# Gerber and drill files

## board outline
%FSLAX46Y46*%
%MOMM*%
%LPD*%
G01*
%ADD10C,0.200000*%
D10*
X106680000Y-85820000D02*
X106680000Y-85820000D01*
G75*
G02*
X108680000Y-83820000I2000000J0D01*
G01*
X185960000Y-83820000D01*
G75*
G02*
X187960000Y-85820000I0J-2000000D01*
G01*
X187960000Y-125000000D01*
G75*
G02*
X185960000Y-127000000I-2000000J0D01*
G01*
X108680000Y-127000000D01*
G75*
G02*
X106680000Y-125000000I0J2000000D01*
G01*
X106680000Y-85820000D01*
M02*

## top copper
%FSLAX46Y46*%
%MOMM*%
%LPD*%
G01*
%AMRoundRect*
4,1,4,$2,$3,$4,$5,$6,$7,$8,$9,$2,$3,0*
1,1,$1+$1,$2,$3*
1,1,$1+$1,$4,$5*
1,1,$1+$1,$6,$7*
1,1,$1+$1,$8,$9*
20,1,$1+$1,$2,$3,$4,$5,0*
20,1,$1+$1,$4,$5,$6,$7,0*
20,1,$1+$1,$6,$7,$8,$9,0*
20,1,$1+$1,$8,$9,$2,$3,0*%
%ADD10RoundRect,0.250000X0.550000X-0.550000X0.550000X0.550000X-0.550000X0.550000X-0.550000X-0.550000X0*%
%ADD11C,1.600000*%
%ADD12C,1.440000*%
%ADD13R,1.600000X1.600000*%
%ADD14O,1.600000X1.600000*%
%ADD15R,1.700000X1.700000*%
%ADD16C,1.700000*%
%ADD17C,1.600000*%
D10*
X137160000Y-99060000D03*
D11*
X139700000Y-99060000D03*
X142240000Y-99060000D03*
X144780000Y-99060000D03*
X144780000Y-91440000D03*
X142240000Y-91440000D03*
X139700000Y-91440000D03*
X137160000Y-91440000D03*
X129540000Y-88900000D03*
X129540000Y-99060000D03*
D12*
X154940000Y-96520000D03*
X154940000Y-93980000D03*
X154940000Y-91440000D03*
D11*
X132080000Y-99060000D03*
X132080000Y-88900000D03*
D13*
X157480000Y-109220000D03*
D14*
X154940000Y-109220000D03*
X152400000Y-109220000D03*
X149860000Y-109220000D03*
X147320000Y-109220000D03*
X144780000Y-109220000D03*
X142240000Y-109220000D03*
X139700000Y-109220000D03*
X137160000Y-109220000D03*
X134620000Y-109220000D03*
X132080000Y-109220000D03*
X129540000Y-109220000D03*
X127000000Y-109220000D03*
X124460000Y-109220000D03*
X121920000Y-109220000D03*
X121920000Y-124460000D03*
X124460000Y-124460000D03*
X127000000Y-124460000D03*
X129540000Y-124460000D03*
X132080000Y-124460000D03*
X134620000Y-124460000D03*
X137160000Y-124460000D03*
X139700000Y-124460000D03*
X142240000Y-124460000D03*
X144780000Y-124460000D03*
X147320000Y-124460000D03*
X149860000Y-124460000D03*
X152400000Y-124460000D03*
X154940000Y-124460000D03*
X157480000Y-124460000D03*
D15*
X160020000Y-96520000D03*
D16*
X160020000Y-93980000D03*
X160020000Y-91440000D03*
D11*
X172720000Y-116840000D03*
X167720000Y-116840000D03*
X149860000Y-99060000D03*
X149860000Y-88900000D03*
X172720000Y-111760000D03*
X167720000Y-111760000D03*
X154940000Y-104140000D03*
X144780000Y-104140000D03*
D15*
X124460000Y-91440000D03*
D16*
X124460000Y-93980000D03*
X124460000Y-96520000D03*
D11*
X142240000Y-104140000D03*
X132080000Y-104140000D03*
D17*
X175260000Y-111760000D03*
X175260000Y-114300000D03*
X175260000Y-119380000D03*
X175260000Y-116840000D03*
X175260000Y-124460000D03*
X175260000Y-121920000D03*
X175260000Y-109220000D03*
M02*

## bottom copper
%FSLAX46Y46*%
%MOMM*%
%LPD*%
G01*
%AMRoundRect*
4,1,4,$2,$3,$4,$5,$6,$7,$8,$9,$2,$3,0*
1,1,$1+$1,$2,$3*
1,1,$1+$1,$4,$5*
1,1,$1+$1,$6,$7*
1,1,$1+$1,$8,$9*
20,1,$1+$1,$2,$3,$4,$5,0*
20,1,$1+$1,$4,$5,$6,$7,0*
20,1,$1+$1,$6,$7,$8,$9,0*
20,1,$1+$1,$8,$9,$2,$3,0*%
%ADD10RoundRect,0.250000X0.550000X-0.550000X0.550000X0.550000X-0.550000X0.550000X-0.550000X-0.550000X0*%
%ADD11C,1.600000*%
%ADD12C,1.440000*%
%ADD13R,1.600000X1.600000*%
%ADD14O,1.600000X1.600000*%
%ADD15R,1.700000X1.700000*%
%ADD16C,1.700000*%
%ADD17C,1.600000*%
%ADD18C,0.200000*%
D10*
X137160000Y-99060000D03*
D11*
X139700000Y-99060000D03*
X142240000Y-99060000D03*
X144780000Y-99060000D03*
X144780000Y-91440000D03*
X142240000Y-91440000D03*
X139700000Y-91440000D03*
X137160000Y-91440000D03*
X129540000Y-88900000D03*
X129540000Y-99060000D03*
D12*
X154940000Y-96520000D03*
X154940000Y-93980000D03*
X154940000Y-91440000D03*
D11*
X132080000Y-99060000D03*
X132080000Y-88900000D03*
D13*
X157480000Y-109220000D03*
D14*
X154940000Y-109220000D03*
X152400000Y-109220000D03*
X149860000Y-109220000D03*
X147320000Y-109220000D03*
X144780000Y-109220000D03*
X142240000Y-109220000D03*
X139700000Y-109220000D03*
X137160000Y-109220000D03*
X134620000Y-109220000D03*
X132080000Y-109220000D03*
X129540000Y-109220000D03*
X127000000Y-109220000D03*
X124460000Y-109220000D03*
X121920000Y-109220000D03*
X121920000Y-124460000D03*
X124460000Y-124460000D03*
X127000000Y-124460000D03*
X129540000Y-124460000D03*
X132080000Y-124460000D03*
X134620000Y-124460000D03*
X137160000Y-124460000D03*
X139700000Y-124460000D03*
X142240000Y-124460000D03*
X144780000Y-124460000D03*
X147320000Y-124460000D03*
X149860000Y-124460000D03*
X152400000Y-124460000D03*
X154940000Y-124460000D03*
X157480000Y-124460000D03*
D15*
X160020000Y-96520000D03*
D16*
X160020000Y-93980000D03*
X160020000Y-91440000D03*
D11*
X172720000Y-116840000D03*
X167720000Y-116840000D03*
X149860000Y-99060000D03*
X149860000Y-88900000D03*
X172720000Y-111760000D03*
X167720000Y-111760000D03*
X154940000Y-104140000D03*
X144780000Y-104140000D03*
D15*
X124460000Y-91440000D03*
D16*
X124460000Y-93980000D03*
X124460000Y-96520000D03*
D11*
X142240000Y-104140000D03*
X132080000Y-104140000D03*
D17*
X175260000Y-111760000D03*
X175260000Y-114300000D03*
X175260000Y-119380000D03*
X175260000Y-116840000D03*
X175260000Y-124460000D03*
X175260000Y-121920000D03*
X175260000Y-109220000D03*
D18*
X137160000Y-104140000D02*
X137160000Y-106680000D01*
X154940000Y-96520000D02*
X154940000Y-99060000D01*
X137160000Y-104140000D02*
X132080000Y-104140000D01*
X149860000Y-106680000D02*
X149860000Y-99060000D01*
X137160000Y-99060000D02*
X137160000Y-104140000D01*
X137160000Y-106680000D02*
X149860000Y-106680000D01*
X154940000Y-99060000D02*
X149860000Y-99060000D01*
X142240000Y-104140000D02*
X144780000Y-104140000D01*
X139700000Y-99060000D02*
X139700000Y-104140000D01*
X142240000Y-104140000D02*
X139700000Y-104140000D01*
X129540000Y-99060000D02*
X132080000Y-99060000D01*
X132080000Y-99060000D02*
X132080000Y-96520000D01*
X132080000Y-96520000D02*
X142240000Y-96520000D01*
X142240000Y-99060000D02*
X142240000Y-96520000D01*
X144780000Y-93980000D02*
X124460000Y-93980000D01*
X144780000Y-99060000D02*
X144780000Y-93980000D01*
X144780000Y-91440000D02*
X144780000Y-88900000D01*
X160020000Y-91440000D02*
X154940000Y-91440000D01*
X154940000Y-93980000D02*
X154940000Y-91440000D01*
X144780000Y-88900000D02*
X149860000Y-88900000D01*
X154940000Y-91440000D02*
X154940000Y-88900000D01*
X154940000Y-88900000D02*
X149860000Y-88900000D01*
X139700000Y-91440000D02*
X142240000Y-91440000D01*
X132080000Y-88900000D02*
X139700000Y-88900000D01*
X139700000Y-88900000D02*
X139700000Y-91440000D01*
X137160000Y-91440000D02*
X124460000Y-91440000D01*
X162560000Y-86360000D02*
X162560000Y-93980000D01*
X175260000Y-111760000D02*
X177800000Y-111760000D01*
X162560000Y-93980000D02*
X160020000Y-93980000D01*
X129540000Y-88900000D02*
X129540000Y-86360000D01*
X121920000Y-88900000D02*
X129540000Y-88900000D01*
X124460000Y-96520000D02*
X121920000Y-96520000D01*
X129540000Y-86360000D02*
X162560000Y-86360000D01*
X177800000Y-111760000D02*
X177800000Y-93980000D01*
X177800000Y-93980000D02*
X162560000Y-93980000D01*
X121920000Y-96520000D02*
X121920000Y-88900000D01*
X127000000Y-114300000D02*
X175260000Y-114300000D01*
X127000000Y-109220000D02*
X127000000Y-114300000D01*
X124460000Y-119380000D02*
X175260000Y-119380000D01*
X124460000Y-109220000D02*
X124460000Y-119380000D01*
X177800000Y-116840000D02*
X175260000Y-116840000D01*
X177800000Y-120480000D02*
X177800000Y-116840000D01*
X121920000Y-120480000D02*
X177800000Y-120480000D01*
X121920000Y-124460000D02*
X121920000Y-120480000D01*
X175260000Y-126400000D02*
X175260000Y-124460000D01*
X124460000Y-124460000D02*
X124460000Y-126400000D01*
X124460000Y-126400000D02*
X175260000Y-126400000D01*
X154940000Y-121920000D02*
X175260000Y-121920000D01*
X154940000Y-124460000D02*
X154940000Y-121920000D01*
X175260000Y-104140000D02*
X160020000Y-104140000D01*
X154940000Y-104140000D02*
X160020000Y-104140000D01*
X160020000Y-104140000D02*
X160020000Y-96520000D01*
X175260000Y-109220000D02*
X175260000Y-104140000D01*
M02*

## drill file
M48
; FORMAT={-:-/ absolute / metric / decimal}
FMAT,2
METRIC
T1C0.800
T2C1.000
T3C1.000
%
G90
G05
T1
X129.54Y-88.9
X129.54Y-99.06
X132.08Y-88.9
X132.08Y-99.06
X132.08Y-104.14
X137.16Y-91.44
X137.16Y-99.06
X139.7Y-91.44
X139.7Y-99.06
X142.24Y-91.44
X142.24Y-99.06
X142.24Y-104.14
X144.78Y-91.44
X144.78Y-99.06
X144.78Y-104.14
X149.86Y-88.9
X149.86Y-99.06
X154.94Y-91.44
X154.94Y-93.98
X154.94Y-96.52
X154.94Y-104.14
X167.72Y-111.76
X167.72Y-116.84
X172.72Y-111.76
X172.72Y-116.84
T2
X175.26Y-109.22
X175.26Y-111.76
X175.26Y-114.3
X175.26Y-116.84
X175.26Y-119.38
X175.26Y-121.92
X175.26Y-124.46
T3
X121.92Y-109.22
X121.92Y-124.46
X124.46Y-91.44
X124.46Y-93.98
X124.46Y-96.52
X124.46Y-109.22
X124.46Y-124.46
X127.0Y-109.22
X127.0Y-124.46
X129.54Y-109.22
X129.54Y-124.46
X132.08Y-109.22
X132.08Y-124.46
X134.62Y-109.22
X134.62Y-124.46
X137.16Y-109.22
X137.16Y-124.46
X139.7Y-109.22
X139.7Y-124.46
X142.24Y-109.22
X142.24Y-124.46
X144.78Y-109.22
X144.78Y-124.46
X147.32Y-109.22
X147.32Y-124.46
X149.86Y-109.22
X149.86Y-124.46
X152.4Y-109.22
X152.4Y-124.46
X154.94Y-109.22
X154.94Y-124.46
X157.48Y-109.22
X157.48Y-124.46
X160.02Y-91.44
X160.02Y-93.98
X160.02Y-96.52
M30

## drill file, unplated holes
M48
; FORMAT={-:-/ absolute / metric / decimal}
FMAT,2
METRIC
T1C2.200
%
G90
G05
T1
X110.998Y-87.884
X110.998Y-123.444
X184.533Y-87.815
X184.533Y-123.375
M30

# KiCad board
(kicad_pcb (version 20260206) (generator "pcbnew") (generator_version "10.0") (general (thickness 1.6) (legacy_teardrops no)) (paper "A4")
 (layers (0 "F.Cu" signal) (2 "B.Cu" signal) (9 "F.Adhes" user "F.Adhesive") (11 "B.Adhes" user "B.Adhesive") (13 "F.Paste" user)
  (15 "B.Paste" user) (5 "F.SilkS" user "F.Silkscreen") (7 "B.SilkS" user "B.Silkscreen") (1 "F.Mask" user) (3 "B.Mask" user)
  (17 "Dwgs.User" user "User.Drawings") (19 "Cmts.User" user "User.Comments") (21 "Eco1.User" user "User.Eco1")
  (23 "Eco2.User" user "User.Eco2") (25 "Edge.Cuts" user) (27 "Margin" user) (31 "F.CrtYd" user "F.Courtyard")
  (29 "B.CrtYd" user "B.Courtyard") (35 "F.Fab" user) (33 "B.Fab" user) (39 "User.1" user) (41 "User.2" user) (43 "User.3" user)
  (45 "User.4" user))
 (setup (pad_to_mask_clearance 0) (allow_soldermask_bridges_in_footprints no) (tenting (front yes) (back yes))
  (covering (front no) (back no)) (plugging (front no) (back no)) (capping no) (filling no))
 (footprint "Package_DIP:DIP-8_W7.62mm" (layer "F.Cu") (at 137.16 99.06 90)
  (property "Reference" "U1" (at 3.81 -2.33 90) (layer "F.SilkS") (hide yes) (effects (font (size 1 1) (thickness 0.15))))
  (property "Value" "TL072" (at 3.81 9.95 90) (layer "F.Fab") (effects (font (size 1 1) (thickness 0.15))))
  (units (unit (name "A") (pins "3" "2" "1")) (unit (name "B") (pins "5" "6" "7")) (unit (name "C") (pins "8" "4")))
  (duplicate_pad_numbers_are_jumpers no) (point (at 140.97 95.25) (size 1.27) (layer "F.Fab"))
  (pad "1" thru_hole roundrect (at 0 0 90) (size 1.6 1.6) (drill 0.8) (layers "*.Cu" "*.Mask") (remove_unused_layers no)
   (roundrect_rratio 0.15625) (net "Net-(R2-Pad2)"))
  (pad "2" thru_hole circle (at 0 2.54 90) (size 1.6 1.6) (drill 0.8) (layers "*.Cu" "*.Mask") (remove_unused_layers no) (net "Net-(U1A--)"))
  (pad "3" thru_hole circle (at 0 5.08 90) (size 1.6 1.6) (drill 0.8) (layers "*.Cu" "*.Mask") (remove_unused_layers no) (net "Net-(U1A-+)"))
  (pad "4" thru_hole circle (at 0 7.62 90) (size 1.6 1.6) (drill 0.8) (layers "*.Cu" "*.Mask") (remove_unused_layers no) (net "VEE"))
  (pad "5" thru_hole circle (at 7.62 7.62 90) (size 1.6 1.6) (drill 0.8) (layers "*.Cu" "*.Mask") (remove_unused_layers no) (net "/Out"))
  (pad "6" thru_hole circle (at 7.62 5.08 90) (size 1.6 1.6) (drill 0.8) (layers "*.Cu" "*.Mask") (remove_unused_layers no)
   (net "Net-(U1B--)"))
  (pad "7" thru_hole circle (at 7.62 2.54 90) (size 1.6 1.6) (drill 0.8) (layers "*.Cu" "*.Mask") (remove_unused_layers no)
   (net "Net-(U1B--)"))
  (pad "8" thru_hole circle (at 7.62 0 90) (size 1.6 1.6) (drill 0.8) (layers "*.Cu" "*.Mask") (remove_unused_layers no) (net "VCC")))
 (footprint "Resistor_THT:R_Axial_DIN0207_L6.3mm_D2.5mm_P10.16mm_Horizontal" (layer "F.Cu") (at 129.54 88.9 -90)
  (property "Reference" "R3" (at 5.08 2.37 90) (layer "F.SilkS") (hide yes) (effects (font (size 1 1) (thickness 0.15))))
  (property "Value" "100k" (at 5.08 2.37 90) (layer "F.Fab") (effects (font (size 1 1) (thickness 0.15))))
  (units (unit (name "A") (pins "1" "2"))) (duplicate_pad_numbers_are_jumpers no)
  (pad "1" thru_hole circle (at 0 0 270) (size 1.6 1.6) (drill 0.8) (layers "*.Cu" "*.Mask") (remove_unused_layers no) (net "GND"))
  (pad "2" thru_hole circle (at 10.16 0 270) (size 1.6 1.6) (drill 0.8) (layers "*.Cu" "*.Mask") (remove_unused_layers no)
   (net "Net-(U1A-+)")))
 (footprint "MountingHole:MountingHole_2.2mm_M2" (layer "F.Cu") (at 110.998 123.444)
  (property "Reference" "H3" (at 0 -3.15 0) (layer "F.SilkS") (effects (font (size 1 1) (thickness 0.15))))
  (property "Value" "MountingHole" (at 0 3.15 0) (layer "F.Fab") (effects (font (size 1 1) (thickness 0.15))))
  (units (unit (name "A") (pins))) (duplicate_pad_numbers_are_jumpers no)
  (pad "" np_thru_hole circle (at 0 0) (size 2.2 2.2) (drill 2.2) (layers "*.Cu" "*.Mask")))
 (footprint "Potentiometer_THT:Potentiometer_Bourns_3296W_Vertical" (layer "F.Cu") (at 154.94 96.52 -90)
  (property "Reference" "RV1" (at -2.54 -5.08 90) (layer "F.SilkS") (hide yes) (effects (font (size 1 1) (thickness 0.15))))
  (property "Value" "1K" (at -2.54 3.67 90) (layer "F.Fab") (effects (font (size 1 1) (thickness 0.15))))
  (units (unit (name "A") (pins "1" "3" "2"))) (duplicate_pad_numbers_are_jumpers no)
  (pad "1" thru_hole circle (at 0 0 270) (size 1.44 1.44) (drill 0.8) (layers "*.Cu" "*.Mask") (remove_unused_layers no)
   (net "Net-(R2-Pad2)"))
  (pad "2" thru_hole circle (at -2.54 0 270) (size 1.44 1.44) (drill 0.8) (layers "*.Cu" "*.Mask") (remove_unused_layers no) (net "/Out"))
  (pad "3" thru_hole circle (at -5.08 0 270) (size 1.44 1.44) (drill 0.8) (layers "*.Cu" "*.Mask") (remove_unused_layers no) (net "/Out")))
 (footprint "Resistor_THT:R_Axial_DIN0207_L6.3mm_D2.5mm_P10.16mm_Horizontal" (layer "F.Cu") (at 132.08 99.06 90)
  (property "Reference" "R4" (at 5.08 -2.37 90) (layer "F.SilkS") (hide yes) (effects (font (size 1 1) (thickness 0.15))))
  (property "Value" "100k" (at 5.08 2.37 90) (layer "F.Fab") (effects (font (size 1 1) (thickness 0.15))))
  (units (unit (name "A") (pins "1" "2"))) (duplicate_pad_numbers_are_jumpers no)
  (pad "1" thru_hole circle (at 0 0 90) (size 1.6 1.6) (drill 0.8) (layers "*.Cu" "*.Mask") (remove_unused_layers no) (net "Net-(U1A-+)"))
  (pad "2" thru_hole circle (at 10.16 0 90) (size 1.6 1.6) (drill 0.8) (layers "*.Cu" "*.Mask") (remove_unused_layers no)
   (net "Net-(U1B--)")))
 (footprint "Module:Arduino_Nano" (layer "F.Cu") (at 157.48 109.22 -90)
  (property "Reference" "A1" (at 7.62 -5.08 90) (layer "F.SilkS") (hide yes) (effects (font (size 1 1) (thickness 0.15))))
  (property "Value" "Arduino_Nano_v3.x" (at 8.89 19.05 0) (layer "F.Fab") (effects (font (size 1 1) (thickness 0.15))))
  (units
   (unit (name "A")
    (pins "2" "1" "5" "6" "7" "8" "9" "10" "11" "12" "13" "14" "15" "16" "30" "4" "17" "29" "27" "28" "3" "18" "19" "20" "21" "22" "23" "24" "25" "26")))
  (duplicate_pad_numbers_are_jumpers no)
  (pad "1" thru_hole rect (at 0 0 270) (size 1.6 1.6) (drill 1) (layers "*.Cu" "*.Mask") (remove_unused_layers no)
   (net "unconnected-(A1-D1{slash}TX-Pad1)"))
  (pad "2" thru_hole oval (at 0 2.54 270) (size 1.6 1.6) (drill 1) (layers "*.Cu" "*.Mask") (remove_unused_layers no)
   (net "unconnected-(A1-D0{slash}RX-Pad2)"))
  (pad "3" thru_hole oval (at 0 5.08 270) (size 1.6 1.6) (drill 1) (layers "*.Cu" "*.Mask") (remove_unused_layers no)
   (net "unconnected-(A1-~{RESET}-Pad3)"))
  (pad "4" thru_hole oval (at 0 7.62 270) (size 1.6 1.6) (drill 1) (layers "*.Cu" "*.Mask") (remove_unused_layers no)
   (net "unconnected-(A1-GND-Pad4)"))
  (pad "5" thru_hole oval (at 0 10.16 270) (size 1.6 1.6) (drill 1) (layers "*.Cu" "*.Mask") (remove_unused_layers no)
   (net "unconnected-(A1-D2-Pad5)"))
  (pad "6" thru_hole oval (at 0 12.7 270) (size 1.6 1.6) (drill 1) (layers "*.Cu" "*.Mask") (remove_unused_layers no)
   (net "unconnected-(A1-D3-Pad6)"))
  (pad "7" thru_hole oval (at 0 15.24 270) (size 1.6 1.6) (drill 1) (layers "*.Cu" "*.Mask") (remove_unused_layers no)
   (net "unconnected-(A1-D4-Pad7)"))
  (pad "8" thru_hole oval (at 0 17.78 270) (size 1.6 1.6) (drill 1) (layers "*.Cu" "*.Mask") (remove_unused_layers no)
   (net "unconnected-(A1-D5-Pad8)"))
  (pad "9" thru_hole oval (at 0 20.32 270) (size 1.6 1.6) (drill 1) (layers "*.Cu" "*.Mask") (remove_unused_layers no)
   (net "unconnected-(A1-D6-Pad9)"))
  (pad "10" thru_hole oval (at 0 22.86 270) (size 1.6 1.6) (drill 1) (layers "*.Cu" "*.Mask") (remove_unused_layers no)
   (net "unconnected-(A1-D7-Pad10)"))
  (pad "11" thru_hole oval (at 0 25.4 270) (size 1.6 1.6) (drill 1) (layers "*.Cu" "*.Mask") (remove_unused_layers no)
   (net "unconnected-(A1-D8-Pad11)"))
  (pad "12" thru_hole oval (at 0 27.94 270) (size 1.6 1.6) (drill 1) (layers "*.Cu" "*.Mask") (remove_unused_layers no)
   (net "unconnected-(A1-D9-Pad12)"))
  (pad "13" thru_hole oval (at 0 30.48 270) (size 1.6 1.6) (drill 1) (layers "*.Cu" "*.Mask") (remove_unused_layers no)
   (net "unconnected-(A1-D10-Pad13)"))
  (pad "14" thru_hole oval (at 0 33.02 270) (size 1.6 1.6) (drill 1) (layers "*.Cu" "*.Mask") (remove_unused_layers no)
   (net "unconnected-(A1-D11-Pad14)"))
  (pad "15" thru_hole oval (at 0 35.56 270) (size 1.6 1.6) (drill 1) (layers "*.Cu" "*.Mask") (remove_unused_layers no)
   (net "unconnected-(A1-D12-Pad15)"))
  (pad "16" thru_hole oval (at 15.24 35.56 270) (size 1.6 1.6) (drill 1) (layers "*.Cu" "*.Mask") (remove_unused_layers no)
   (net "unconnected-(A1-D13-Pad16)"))
  (pad "17" thru_hole oval (at 15.24 33.02 270) (size 1.6 1.6) (drill 1) (layers "*.Cu" "*.Mask") (remove_unused_layers no)
   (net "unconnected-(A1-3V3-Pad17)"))
  (pad "18" thru_hole oval (at 15.24 30.48 270) (size 1.6 1.6) (drill 1) (layers "*.Cu" "*.Mask") (remove_unused_layers no)
   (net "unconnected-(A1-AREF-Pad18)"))
  (pad "19" thru_hole oval (at 15.24 27.94 270) (size 1.6 1.6) (drill 1) (layers "*.Cu" "*.Mask") (remove_unused_layers no)
   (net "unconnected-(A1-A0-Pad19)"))
  (pad "20" thru_hole oval (at 15.24 25.4 270) (size 1.6 1.6) (drill 1) (layers "*.Cu" "*.Mask") (remove_unused_layers no)
   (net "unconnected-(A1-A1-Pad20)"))
  (pad "21" thru_hole oval (at 15.24 22.86 270) (size 1.6 1.6) (drill 1) (layers "*.Cu" "*.Mask") (remove_unused_layers no)
   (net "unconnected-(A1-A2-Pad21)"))
  (pad "22" thru_hole oval (at 15.24 20.32 270) (size 1.6 1.6) (drill 1) (layers "*.Cu" "*.Mask") (remove_unused_layers no)
   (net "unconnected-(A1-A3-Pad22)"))
  (pad "23" thru_hole oval (at 15.24 17.78 270) (size 1.6 1.6) (drill 1) (layers "*.Cu" "*.Mask") (remove_unused_layers no)
   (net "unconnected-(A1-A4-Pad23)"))
  (pad "24" thru_hole oval (at 15.24 15.24 270) (size 1.6 1.6) (drill 1) (layers "*.Cu" "*.Mask") (remove_unused_layers no)
   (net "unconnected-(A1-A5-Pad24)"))
  (pad "25" thru_hole oval (at 15.24 12.7 270) (size 1.6 1.6) (drill 1) (layers "*.Cu" "*.Mask") (remove_unused_layers no)
   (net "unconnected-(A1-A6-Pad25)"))
  (pad "26" thru_hole oval (at 15.24 10.16 270) (size 1.6 1.6) (drill 1) (layers "*.Cu" "*.Mask") (remove_unused_layers no)
   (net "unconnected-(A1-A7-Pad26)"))
  (pad "27" thru_hole oval (at 15.24 7.62 270) (size 1.6 1.6) (drill 1) (layers "*.Cu" "*.Mask") (remove_unused_layers no)
   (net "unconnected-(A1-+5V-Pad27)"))
  (pad "28" thru_hole oval (at 15.24 5.08 270) (size 1.6 1.6) (drill 1) (layers "*.Cu" "*.Mask") (remove_unused_layers no)
   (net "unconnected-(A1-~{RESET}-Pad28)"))
  (pad "29" thru_hole oval (at 15.24 2.54 270) (size 1.6 1.6) (drill 1) (layers "*.Cu" "*.Mask") (remove_unused_layers no)
   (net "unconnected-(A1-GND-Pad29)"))
  (pad "30" thru_hole oval (at 15.24 0 270) (size 1.6 1.6) (drill 1) (layers "*.Cu" "*.Mask") (remove_unused_layers no)
   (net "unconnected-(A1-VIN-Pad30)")))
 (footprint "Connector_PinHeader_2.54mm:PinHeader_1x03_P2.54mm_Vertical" (layer "F.Cu") (at 160.02 96.52 180)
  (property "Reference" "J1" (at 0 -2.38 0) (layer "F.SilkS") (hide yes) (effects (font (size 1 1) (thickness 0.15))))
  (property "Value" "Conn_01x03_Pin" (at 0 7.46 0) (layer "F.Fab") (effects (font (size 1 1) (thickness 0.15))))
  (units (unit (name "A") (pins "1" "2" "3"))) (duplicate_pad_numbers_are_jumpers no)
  (pad "1" thru_hole rect (at 0 0 180) (size 1.7 1.7) (drill 1) (layers "*.Cu" "*.Mask") (remove_unused_layers no) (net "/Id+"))
  (pad "2" thru_hole circle (at 0 2.54 180) (size 1.7 1.7) (drill 1) (layers "*.Cu" "*.Mask") (remove_unused_layers no) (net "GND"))
  (pad "3" thru_hole circle (at 0 5.08 180) (size 1.7 1.7) (drill 1) (layers "*.Cu" "*.Mask") (remove_unused_layers no) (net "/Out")))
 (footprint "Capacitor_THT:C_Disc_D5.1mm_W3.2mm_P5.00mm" (layer "F.Cu") (at 172.72 116.84 180)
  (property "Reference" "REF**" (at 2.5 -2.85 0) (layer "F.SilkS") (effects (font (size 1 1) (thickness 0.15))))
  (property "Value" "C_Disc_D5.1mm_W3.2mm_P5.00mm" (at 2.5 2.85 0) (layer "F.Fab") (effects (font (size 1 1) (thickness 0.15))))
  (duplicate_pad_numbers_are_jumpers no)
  (pad "1" thru_hole circle (at 0 0 180) (size 1.6 1.6) (drill 0.8) (layers "*.Cu" "*.Mask") (remove_unused_layers no))
  (pad "2" thru_hole circle (at 5 0 180) (size 1.6 1.6) (drill 0.8) (layers "*.Cu" "*.Mask") (remove_unused_layers no)))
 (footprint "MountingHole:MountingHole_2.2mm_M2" (layer "F.Cu") (at 184.533168 87.815138)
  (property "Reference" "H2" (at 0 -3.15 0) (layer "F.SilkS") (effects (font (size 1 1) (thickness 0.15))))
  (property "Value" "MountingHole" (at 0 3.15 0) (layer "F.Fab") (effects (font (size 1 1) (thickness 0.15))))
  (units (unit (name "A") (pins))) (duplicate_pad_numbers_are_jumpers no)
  (pad "" np_thru_hole circle (at 0 0) (size 2.2 2.2) (drill 2.2) (layers "*.Cu" "*.Mask")))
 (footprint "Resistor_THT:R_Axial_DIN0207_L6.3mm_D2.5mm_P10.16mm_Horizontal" (layer "F.Cu") (at 149.86 99.06 90)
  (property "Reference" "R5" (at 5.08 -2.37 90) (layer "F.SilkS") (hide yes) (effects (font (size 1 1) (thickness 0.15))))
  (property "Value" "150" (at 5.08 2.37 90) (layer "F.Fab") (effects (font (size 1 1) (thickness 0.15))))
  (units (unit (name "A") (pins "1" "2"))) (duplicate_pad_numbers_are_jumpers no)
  (pad "1" thru_hole circle (at 0 0 90) (size 1.6 1.6) (drill 0.8) (layers "*.Cu" "*.Mask") (remove_unused_layers no) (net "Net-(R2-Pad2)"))
  (pad "2" thru_hole circle (at 10.16 0 90) (size 1.6 1.6) (drill 0.8) (layers "*.Cu" "*.Mask") (remove_unused_layers no) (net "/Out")))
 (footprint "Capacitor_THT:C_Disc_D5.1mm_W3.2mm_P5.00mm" (layer "F.Cu") (at 172.72 111.76 180)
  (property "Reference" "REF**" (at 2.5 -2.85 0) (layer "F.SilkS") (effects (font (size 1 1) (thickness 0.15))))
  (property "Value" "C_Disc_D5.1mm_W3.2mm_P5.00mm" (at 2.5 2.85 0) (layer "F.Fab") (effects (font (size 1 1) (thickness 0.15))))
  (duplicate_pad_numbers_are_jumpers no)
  (pad "1" thru_hole circle (at 0 0 180) (size 1.6 1.6) (drill 0.8) (layers "*.Cu" "*.Mask") (remove_unused_layers no))
  (pad "2" thru_hole circle (at 5 0 180) (size 1.6 1.6) (drill 0.8) (layers "*.Cu" "*.Mask") (remove_unused_layers no)))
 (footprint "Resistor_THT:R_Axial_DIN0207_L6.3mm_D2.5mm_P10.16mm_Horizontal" (layer "F.Cu") (at 154.94 104.14 180)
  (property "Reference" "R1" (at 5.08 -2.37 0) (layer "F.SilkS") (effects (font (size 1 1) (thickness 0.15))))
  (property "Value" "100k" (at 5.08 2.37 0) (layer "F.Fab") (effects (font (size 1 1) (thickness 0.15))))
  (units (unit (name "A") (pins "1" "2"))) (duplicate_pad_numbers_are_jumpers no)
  (pad "1" thru_hole circle (at 0 0 180) (size 1.6 1.6) (drill 0.8) (layers "*.Cu" "*.Mask") (remove_unused_layers no) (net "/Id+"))
  (pad "2" thru_hole circle (at 10.16 0 180) (size 1.6 1.6) (drill 0.8) (layers "*.Cu" "*.Mask") (remove_unused_layers no)
   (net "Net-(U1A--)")))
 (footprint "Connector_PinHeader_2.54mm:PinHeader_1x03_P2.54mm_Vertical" (layer "F.Cu") (at 124.46 91.44)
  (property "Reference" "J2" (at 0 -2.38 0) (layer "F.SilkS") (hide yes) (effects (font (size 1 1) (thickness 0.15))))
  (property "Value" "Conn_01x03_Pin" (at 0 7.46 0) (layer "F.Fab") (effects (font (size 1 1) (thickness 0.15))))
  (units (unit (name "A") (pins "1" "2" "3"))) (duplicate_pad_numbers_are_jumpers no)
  (pad "1" thru_hole rect (at 0 0) (size 1.7 1.7) (drill 1) (layers "*.Cu" "*.Mask") (remove_unused_layers no) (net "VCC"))
  (pad "2" thru_hole circle (at 0 2.54) (size 1.7 1.7) (drill 1) (layers "*.Cu" "*.Mask") (remove_unused_layers no) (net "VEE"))
  (pad "3" thru_hole circle (at 0 5.08) (size 1.7 1.7) (drill 1) (layers "*.Cu" "*.Mask") (remove_unused_layers no) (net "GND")))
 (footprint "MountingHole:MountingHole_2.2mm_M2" (layer "F.Cu") (at 184.533168 123.375138)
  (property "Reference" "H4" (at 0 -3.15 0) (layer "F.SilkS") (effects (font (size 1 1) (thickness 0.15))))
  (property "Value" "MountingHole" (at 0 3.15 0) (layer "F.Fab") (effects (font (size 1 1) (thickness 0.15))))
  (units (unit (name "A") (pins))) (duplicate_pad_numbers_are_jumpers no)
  (pad "" np_thru_hole circle (at 0 0) (size 2.2 2.2) (drill 2.2) (layers "*.Cu" "*.Mask")))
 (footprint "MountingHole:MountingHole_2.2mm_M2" (layer "F.Cu") (at 110.998 87.884)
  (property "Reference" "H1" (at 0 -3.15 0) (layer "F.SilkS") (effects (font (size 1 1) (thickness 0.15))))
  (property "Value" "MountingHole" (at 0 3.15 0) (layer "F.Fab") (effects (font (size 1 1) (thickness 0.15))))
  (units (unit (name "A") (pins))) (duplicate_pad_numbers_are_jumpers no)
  (pad "" np_thru_hole circle (at 0 0) (size 2.2 2.2) (drill 2.2) (layers "*.Cu" "*.Mask")))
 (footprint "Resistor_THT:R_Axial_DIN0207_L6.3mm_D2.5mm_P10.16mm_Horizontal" (layer "F.Cu") (at 142.24 104.14 180)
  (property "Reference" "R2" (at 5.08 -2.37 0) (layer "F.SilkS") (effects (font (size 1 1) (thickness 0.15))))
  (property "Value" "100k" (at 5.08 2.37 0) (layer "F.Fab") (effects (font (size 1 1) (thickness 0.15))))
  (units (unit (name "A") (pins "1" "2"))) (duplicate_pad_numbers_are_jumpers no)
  (pad "1" thru_hole circle (at 0 0 180) (size 1.6 1.6) (drill 0.8) (layers "*.Cu" "*.Mask") (remove_unused_layers no) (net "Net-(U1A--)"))
  (pad "2" thru_hole circle (at 10.16 0 180) (size 1.6 1.6) (drill 0.8) (layers "*.Cu" "*.Mask") (remove_unused_layers no)
   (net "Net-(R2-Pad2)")))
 (gr_rect (start 106.68 83.82) (end 187.96 127) (radius 2) (stroke (width 0.2) (type solid)) (fill no) (layer "Edge.Cuts"))
 (segment (start 137.16 104.14) (end 137.16 106.68) (width 0.2) (layer "B.Cu") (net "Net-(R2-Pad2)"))
 (segment (start 154.94 96.52) (end 154.94 99.06) (width 0.2) (layer "B.Cu") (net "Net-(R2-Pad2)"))
 (segment (start 137.16 104.14) (end 132.08 104.14) (width 0.2) (layer "B.Cu") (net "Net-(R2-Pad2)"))
 (segment (start 149.86 106.68) (end 149.86 99.06) (width 0.2) (layer "B.Cu") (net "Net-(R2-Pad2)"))
 (segment (start 137.16 99.06) (end 137.16 104.14) (width 0.2) (layer "B.Cu") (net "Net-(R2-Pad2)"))
 (segment (start 137.16 106.68) (end 149.86 106.68) (width 0.2) (layer "B.Cu") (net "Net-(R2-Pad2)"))
 (segment (start 154.94 99.06) (end 149.86 99.06) (width 0.2) (layer "B.Cu") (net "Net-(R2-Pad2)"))
 (segment (start 142.24 104.14) (end 144.78 104.14) (width 0.2) (layer "B.Cu") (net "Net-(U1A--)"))
 (segment (start 139.7 99.06) (end 139.7 104.14) (width 0.2) (layer "B.Cu") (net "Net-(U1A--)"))
 (segment (start 142.24 104.14) (end 139.7 104.14) (width 0.2) (layer "B.Cu") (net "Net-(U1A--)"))
 (segment (start 129.54 99.06) (end 132.08 99.06) (width 0.2) (layer "B.Cu") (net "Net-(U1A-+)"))
 (segment (start 132.08 99.06) (end 132.08 96.52) (width 0.2) (layer "B.Cu") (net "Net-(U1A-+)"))
 (segment (start 132.08 96.52) (end 142.24 96.52) (width 0.2) (layer "B.Cu") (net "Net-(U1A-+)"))
 (segment (start 142.24 99.06) (end 142.24 96.52) (width 0.2) (layer "B.Cu") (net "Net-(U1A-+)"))
 (segment (start 144.78 93.98) (end 124.46 93.98) (width 0.2) (layer "B.Cu") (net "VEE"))
 (segment (start 144.78 99.06) (end 144.78 93.98) (width 0.2) (layer "B.Cu") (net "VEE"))
 (segment (start 144.78 91.44) (end 144.78 88.9) (width 0.2) (layer "B.Cu") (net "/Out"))
 (segment (start 160.02 91.44) (end 154.94 91.44) (width 0.2) (layer "B.Cu") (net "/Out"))
 (segment (start 154.94 93.98) (end 154.94 91.44) (width 0.2) (layer "B.Cu") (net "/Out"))
 (segment (start 144.78 88.9) (end 149.86 88.9) (width 0.2) (layer "B.Cu") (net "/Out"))
 (segment (start 154.94 91.44) (end 154.94 88.9) (width 0.2) (layer "B.Cu") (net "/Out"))
 (segment (start 154.94 88.9) (end 149.86 88.9) (width 0.2) (layer "B.Cu") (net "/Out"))
 (segment (start 139.7 91.44) (end 142.24 91.44) (width 0.2) (layer "B.Cu") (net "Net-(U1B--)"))
 (segment (start 132.08 88.9) (end 139.7 88.9) (width 0.2) (layer "B.Cu") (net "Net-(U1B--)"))
 (segment (start 139.7 88.9) (end 139.7 91.44) (width 0.2) (layer "B.Cu") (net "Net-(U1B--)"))
 (segment (start 137.16 91.44) (end 124.46 91.44) (width 0.2) (layer "B.Cu") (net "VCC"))
 (via (at 175.26 111.76) (size 1.6) (drill 1) (layers "F.Cu" "B.Cu") (free yes) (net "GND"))
 (segment (start 162.56 86.36) (end 162.56 93.98) (width 0.2) (layer "B.Cu") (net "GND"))
 (segment (start 175.26 111.76) (end 177.8 111.76) (width 0.2) (layer "B.Cu") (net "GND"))
 (segment (start 162.56 93.98) (end 160.02 93.98) (width 0.2) (layer "B.Cu") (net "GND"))
 (segment (start 129.54 88.9) (end 129.54 86.36) (width 0.2) (layer "B.Cu") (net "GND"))
 (segment (start 121.92 88.9) (end 129.54 88.9) (width 0.2) (layer "B.Cu") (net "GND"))
 (segment (start 124.46 96.52) (end 121.92 96.52) (width 0.2) (layer "B.Cu") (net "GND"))
 (segment (start 129.54 86.36) (end 162.56 86.36) (width 0.2) (layer "B.Cu") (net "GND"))
 (segment (start 177.8 111.76) (end 177.8 93.98) (width 0.2) (layer "B.Cu") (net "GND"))
 (segment (start 177.8 93.98) (end 162.56 93.98) (width 0.2) (layer "B.Cu") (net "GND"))
 (segment (start 121.92 96.52) (end 121.92 88.9) (width 0.2) (layer "B.Cu") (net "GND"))
 (via (at 175.26 114.3) (size 1.6) (drill 1) (layers "F.Cu" "B.Cu") (free yes) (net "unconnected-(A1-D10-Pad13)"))
 (segment (start 127 114.3) (end 175.26 114.3) (width 0.2) (layer "B.Cu") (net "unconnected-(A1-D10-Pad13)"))
 (segment (start 127 109.22) (end 127 114.3) (width 0.2) (layer "B.Cu") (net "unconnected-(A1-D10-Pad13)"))
 (via (at 175.26 119.38) (size 1.6) (drill 1) (layers "F.Cu" "B.Cu") (free yes) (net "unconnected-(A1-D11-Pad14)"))
 (segment (start 124.46 119.38) (end 175.26 119.38) (width 0.2) (layer "B.Cu") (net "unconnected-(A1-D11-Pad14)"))
 (segment (start 124.46 109.22) (end 124.46 119.38) (width 0.2) (layer "B.Cu") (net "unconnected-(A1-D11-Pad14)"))
 (via (at 175.26 116.84) (size 1.6) (drill 1) (layers "F.Cu" "B.Cu") (free yes) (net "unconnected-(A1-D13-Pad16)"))
 (segment (start 177.8 116.84) (end 175.26 116.84) (width 0.2) (layer "B.Cu") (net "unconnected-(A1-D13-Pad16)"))
 (segment (start 177.8 120.48) (end 177.8 116.84) (width 0.2) (layer "B.Cu") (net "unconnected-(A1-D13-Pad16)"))
 (segment (start 121.92 120.48) (end 177.8 120.48) (width 0.2) (layer "B.Cu") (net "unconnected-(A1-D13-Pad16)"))
 (segment (start 121.92 124.46) (end 121.92 120.48) (width 0.2) (layer "B.Cu") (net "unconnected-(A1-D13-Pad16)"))
 (via (at 175.26 124.46) (size 1.6) (drill 1) (layers "F.Cu" "B.Cu") (free yes) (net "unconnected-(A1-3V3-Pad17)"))
 (segment (start 175.26 126.4) (end 175.26 124.46) (width 0.2) (layer "B.Cu") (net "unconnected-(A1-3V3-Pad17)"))
 (segment (start 124.46 124.46) (end 124.46 126.4) (width 0.2) (layer "B.Cu") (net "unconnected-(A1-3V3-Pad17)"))
 (segment (start 124.46 126.4) (end 175.26 126.4) (width 0.2) (layer "B.Cu") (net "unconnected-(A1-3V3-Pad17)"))
 (via (at 175.26 121.92) (size 1.6) (drill 1) (layers "F.Cu" "B.Cu") (free yes) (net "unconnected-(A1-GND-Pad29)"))
 (segment (start 154.94 121.92) (end 175.26 121.92) (width 0.2) (layer "B.Cu") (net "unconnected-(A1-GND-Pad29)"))
 (segment (start 154.94 124.46) (end 154.94 121.92) (width 0.2) (layer "B.Cu") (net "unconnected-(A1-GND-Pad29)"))
 (via (at 175.26 109.22) (size 1.6) (drill 1) (layers "F.Cu" "B.Cu") (free yes) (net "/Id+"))
 (segment (start 175.26 104.14) (end 160.02 104.14) (width 0.2) (layer "B.Cu") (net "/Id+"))
 (segment (start 154.94 104.14) (end 160.02 104.14) (width 0.2) (layer "B.Cu") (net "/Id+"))
 (segment (start 160.02 104.14) (end 160.02 96.52) (width 0.2) (layer "B.Cu") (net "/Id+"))
 (segment (start 175.26 109.22) (end 175.26 104.14) (width 0.2) (layer "B.Cu") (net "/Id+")))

